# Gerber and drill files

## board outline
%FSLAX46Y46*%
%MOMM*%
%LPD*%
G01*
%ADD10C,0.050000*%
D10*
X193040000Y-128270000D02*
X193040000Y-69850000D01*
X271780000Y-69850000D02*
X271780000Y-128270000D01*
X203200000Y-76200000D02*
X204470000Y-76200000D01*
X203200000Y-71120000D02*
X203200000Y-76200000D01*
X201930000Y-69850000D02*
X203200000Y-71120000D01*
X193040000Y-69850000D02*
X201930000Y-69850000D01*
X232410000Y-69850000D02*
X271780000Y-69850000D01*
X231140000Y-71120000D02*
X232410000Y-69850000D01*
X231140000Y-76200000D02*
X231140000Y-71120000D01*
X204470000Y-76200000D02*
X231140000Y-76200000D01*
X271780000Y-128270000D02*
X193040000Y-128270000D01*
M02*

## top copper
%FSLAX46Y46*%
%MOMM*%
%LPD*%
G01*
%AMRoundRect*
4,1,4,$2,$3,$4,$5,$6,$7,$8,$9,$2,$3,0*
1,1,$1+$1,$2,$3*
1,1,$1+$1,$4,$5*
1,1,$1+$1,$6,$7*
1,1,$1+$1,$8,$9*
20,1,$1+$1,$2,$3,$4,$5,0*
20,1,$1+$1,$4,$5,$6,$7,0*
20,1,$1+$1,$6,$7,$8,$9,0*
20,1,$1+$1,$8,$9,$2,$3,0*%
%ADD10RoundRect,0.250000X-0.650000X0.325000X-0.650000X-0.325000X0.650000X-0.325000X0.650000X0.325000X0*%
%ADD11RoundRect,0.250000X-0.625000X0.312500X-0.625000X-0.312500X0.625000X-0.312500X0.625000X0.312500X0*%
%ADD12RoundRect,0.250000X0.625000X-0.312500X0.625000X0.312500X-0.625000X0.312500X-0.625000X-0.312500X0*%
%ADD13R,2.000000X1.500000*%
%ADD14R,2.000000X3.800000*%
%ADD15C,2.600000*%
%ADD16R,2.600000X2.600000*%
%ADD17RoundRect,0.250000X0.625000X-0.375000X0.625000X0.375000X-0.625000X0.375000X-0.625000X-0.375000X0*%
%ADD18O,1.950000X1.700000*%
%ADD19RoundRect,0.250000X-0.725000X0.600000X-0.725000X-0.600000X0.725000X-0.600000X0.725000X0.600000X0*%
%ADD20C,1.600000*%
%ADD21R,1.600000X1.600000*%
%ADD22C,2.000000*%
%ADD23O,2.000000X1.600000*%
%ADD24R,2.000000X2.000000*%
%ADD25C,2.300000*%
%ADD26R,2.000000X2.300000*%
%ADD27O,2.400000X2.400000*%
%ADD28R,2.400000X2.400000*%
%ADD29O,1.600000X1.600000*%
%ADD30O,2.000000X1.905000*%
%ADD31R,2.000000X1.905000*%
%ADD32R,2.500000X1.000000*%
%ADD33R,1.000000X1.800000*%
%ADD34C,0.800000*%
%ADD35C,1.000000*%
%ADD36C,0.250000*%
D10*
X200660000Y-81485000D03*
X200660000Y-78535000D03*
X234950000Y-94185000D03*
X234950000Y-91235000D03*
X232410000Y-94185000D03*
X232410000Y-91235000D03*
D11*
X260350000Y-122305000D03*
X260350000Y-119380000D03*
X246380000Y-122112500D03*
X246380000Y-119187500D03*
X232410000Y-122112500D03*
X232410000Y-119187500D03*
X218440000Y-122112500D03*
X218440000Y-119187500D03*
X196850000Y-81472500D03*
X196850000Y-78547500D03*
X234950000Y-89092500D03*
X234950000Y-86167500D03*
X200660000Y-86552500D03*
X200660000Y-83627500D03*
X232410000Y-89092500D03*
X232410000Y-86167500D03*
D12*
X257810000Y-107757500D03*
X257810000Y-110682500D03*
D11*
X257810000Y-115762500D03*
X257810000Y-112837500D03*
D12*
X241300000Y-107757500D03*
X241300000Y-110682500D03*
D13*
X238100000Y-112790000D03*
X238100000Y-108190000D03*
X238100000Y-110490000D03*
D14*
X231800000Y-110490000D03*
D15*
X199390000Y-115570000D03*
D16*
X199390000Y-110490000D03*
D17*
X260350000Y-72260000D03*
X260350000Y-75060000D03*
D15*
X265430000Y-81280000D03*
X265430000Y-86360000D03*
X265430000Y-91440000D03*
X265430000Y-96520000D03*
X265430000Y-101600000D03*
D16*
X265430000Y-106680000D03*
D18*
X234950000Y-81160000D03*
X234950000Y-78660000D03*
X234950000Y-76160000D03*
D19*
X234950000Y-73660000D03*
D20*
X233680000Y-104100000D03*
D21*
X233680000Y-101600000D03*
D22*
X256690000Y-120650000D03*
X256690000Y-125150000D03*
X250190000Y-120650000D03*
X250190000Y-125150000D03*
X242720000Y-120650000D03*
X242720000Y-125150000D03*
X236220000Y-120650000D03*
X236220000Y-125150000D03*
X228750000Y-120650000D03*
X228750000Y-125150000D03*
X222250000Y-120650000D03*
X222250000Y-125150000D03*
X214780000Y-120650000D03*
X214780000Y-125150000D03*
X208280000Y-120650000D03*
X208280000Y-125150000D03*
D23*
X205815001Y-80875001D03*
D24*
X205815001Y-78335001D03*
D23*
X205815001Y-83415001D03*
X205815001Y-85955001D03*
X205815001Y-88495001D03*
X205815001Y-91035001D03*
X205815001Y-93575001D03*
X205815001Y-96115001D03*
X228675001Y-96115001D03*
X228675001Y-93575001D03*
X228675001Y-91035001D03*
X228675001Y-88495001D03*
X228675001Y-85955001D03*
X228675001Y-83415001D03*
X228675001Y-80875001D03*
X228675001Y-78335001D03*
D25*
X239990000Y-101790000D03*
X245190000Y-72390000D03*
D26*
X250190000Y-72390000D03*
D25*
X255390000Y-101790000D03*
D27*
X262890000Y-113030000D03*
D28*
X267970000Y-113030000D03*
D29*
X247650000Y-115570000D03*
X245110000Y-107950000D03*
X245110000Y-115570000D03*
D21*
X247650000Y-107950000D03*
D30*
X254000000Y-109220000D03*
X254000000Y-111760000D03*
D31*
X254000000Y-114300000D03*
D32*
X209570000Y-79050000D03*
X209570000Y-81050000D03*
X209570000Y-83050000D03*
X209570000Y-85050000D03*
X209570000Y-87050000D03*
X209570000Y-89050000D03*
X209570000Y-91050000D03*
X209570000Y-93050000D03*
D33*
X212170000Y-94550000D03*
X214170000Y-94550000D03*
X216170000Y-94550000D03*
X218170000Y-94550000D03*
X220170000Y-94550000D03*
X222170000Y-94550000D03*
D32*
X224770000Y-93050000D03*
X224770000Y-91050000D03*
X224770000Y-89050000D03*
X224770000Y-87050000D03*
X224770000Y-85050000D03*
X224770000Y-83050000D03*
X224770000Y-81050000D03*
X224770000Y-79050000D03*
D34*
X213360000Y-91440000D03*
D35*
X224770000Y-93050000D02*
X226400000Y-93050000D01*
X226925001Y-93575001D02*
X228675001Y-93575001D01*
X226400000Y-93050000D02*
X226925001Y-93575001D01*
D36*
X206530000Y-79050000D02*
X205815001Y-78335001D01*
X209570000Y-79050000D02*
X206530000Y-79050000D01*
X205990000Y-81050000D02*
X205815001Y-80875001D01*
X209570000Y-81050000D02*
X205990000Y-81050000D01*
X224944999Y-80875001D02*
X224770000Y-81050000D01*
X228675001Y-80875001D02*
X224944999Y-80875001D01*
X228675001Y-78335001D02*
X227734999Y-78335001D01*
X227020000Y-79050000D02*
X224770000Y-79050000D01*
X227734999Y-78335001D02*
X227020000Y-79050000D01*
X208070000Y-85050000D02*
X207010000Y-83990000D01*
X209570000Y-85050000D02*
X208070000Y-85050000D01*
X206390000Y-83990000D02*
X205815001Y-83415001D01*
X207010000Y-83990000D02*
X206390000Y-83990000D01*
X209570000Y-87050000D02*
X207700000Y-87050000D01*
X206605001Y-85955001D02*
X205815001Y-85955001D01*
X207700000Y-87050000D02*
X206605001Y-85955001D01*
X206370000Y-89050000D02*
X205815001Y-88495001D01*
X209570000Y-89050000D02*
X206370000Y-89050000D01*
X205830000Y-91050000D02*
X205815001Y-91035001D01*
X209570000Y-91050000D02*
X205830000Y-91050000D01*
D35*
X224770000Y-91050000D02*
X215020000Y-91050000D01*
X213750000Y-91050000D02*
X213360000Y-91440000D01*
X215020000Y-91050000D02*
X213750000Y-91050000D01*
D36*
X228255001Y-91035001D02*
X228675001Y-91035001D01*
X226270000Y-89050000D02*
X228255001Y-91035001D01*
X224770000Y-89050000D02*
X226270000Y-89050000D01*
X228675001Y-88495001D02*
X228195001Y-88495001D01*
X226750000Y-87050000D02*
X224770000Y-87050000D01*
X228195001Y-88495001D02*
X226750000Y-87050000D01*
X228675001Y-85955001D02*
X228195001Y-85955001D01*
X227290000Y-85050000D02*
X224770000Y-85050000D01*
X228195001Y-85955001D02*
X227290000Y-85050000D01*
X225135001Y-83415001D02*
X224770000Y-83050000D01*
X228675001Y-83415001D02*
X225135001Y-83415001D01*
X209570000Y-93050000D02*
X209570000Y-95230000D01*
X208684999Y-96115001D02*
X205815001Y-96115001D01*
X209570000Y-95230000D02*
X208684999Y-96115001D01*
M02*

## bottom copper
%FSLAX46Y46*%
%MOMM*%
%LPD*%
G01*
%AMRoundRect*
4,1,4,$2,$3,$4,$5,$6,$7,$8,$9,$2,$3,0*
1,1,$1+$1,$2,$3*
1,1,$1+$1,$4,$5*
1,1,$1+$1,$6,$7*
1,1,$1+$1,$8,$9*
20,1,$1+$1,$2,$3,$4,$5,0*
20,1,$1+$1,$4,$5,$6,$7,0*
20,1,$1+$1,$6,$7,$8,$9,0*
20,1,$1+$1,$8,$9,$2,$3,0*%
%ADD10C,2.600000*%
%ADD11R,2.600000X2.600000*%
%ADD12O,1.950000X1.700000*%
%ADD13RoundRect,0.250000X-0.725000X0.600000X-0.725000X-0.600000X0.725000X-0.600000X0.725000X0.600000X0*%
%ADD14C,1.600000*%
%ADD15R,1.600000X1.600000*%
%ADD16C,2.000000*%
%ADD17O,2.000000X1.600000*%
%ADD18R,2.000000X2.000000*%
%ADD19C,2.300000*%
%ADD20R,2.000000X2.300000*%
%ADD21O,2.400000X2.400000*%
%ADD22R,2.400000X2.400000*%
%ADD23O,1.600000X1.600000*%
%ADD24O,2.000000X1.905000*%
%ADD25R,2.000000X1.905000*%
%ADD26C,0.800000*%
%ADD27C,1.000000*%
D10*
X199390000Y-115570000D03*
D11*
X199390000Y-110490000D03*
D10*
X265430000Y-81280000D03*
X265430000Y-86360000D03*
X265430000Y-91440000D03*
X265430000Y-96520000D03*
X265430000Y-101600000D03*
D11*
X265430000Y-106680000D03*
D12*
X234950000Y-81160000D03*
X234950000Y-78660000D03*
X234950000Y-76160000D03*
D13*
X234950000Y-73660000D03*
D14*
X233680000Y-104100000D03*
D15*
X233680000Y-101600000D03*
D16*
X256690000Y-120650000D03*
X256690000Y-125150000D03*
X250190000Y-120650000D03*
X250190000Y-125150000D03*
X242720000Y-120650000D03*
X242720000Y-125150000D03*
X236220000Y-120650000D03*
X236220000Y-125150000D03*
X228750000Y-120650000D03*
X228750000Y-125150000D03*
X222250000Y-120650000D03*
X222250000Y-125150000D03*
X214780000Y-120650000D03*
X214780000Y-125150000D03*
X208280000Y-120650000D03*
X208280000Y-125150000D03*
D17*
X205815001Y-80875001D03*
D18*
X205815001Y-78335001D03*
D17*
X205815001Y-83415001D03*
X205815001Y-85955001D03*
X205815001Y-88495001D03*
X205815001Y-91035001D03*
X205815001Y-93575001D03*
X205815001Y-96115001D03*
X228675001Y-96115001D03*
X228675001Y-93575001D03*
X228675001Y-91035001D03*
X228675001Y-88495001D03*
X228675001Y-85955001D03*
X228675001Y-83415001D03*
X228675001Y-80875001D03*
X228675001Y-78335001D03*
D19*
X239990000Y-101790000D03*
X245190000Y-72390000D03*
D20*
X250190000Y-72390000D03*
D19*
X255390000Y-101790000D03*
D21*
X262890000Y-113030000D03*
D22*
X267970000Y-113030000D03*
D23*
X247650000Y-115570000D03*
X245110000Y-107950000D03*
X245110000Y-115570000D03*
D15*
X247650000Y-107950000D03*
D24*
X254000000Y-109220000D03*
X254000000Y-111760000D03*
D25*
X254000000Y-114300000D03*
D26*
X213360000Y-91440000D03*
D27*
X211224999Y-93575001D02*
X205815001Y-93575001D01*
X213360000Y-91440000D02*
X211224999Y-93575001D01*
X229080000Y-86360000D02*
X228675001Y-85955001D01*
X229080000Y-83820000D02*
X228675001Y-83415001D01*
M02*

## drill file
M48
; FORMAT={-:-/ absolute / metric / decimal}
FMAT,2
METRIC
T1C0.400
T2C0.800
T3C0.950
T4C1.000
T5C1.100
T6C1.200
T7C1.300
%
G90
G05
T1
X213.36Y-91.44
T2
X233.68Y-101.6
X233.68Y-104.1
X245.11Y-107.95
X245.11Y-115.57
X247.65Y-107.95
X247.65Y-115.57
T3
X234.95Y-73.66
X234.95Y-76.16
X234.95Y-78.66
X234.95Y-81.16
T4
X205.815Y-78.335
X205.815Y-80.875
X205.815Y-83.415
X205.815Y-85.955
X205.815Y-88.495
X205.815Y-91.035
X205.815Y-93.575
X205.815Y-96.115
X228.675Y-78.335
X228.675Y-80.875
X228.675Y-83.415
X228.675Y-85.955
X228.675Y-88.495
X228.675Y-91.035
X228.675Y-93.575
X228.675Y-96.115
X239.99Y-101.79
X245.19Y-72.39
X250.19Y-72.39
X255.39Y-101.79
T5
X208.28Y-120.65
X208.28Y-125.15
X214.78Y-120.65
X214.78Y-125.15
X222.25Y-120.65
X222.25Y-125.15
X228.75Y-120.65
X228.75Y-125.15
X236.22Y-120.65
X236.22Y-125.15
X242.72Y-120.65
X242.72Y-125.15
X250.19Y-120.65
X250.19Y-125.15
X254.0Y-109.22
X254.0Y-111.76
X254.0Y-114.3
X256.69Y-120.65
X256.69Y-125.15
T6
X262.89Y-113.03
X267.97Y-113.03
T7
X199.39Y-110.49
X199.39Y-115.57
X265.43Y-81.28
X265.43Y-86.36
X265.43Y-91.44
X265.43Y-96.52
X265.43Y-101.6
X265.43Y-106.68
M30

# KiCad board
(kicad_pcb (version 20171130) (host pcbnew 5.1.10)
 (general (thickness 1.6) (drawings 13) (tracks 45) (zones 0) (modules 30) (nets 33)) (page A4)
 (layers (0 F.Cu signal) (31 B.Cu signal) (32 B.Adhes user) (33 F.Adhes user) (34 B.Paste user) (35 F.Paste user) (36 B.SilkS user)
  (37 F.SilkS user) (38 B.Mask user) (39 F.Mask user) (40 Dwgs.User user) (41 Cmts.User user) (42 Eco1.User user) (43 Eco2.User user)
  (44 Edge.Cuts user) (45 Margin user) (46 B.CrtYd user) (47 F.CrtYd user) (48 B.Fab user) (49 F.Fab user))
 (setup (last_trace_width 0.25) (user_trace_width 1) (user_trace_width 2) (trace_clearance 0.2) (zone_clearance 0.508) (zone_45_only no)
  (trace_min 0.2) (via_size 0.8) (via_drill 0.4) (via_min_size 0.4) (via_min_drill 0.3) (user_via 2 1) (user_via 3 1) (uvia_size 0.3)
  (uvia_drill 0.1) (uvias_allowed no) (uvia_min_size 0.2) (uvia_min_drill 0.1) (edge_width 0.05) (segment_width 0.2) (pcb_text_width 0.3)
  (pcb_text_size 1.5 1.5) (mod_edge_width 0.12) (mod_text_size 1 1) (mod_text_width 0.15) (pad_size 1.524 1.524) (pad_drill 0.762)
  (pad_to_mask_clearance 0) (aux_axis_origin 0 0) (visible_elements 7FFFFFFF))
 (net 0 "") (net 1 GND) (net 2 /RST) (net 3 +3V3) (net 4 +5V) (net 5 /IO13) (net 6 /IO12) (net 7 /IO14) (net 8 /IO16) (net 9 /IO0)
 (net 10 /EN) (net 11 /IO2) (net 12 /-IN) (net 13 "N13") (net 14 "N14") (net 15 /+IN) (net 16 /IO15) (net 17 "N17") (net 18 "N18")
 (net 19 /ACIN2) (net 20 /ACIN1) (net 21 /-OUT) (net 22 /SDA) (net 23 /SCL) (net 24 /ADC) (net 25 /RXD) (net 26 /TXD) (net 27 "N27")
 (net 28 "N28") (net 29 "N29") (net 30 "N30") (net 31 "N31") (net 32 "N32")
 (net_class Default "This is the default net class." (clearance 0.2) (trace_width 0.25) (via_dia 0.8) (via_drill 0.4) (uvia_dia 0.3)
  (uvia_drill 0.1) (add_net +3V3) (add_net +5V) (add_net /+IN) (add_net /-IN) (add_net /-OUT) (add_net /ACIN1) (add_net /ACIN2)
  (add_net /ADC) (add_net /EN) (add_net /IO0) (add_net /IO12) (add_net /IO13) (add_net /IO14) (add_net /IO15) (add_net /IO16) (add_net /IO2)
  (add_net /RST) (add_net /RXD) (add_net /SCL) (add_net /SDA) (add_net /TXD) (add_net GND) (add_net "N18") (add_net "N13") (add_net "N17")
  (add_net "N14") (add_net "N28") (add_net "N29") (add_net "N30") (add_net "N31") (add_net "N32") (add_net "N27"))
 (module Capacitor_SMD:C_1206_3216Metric (layer F.Cu) (at 200.66 80.01 270)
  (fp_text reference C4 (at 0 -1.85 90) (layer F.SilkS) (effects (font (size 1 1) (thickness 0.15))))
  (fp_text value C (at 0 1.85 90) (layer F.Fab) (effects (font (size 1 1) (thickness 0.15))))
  (pad 2 smd roundrect (at 1.475 0 270) (size 1.15 1.8) (layers F.Cu F.Paste F.Mask) (roundrect_rratio 0.217391) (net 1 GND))
  (pad 1 smd roundrect (at -1.475 0 270) (size 1.15 1.8) (layers F.Cu F.Paste F.Mask) (roundrect_rratio 0.217391) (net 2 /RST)))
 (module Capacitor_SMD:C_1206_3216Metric (layer F.Cu) (at 234.95 92.71 270)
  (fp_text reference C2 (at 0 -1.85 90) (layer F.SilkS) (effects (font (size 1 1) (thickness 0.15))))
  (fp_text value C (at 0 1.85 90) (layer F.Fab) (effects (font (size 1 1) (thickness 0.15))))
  (pad 2 smd roundrect (at 1.475 0 270) (size 1.15 1.8) (layers F.Cu F.Paste F.Mask) (roundrect_rratio 0.217391) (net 1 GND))
  (pad 1 smd roundrect (at -1.475 0 270) (size 1.15 1.8) (layers F.Cu F.Paste F.Mask) (roundrect_rratio 0.217391) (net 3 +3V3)))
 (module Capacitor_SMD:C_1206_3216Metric (layer F.Cu) (at 232.41 92.71 270)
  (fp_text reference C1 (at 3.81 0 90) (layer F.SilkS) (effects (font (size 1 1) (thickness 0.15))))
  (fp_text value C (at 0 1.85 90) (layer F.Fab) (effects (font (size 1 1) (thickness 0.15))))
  (pad 2 smd roundrect (at 1.475 0 270) (size 1.15 1.8) (layers F.Cu F.Paste F.Mask) (roundrect_rratio 0.217391) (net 1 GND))
  (pad 1 smd roundrect (at -1.475 0 270) (size 1.15 1.8) (layers F.Cu F.Paste F.Mask) (roundrect_rratio 0.217391) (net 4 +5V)))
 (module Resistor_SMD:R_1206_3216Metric (layer F.Cu) (at 260.35 120.8425 270)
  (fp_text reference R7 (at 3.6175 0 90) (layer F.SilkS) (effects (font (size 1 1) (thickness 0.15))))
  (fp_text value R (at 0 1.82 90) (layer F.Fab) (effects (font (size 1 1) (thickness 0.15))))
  (pad 2 smd roundrect (at 1.4625 0 270) (size 1.125 1.75) (layers F.Cu F.Paste F.Mask) (roundrect_rratio 0.222222) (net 1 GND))
  (pad 1 smd roundrect (at -1.4625 0 270) (size 1.125 1.75) (layers F.Cu F.Paste F.Mask) (roundrect_rratio 0.222222) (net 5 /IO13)))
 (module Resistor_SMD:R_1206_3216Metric (layer F.Cu) (at 246.38 120.65 270)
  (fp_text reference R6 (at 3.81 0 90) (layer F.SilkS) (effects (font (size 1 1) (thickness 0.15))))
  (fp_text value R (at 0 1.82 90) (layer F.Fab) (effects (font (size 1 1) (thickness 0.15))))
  (pad 2 smd roundrect (at 1.4625 0 270) (size 1.125 1.75) (layers F.Cu F.Paste F.Mask) (roundrect_rratio 0.222222) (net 1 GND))
  (pad 1 smd roundrect (at -1.4625 0 270) (size 1.125 1.75) (layers F.Cu F.Paste F.Mask) (roundrect_rratio 0.222222) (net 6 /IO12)))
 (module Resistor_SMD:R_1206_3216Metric (layer F.Cu) (at 232.41 120.65 270)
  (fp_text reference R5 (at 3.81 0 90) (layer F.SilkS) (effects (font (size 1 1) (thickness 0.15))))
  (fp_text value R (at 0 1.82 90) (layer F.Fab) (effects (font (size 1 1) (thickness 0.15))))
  (pad 2 smd roundrect (at 1.4625 0 270) (size 1.125 1.75) (layers F.Cu F.Paste F.Mask) (roundrect_rratio 0.222222) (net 1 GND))
  (pad 1 smd roundrect (at -1.4625 0 270) (size 1.125 1.75) (layers F.Cu F.Paste F.Mask) (roundrect_rratio 0.222222) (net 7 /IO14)))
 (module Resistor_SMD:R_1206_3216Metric (layer F.Cu) (at 218.44 120.65 270)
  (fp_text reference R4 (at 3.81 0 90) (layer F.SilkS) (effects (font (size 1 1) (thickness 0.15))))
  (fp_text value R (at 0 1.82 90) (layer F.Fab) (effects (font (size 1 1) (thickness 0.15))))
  (pad 2 smd roundrect (at 1.4625 0 270) (size 1.125 1.75) (layers F.Cu F.Paste F.Mask) (roundrect_rratio 0.222222) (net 1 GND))
  (pad 1 smd roundrect (at -1.4625 0 270) (size 1.125 1.75) (layers F.Cu F.Paste F.Mask) (roundrect_rratio 0.222222) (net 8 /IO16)))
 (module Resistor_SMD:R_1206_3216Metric (layer F.Cu) (at 196.85 80.01 270)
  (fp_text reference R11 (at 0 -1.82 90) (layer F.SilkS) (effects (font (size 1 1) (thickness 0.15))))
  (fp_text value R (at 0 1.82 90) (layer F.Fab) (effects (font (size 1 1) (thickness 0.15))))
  (pad 2 smd roundrect (at 1.4625 0 270) (size 1.125 1.75) (layers F.Cu F.Paste F.Mask) (roundrect_rratio 0.222222) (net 3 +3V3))
  (pad 1 smd roundrect (at -1.4625 0 270) (size 1.125 1.75) (layers F.Cu F.Paste F.Mask) (roundrect_rratio 0.222222) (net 2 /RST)))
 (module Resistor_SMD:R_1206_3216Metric (layer F.Cu) (at 234.95 87.63 270)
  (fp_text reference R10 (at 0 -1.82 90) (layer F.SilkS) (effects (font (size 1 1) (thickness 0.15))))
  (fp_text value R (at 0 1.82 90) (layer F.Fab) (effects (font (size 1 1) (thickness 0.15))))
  (pad 2 smd roundrect (at 1.4625 0 270) (size 1.125 1.75) (layers F.Cu F.Paste F.Mask) (roundrect_rratio 0.222222) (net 3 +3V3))
  (pad 1 smd roundrect (at -1.4625 0 270) (size 1.125 1.75) (layers F.Cu F.Paste F.Mask) (roundrect_rratio 0.222222) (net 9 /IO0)))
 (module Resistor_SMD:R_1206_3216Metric (layer F.Cu) (at 200.66 85.09 270)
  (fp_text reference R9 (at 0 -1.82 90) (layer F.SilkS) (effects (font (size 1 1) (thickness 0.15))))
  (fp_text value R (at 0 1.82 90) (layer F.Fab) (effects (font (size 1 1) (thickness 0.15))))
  (pad 2 smd roundrect (at 1.4625 0 270) (size 1.125 1.75) (layers F.Cu F.Paste F.Mask) (roundrect_rratio 0.222222) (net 3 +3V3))
  (pad 1 smd roundrect (at -1.4625 0 270) (size 1.125 1.75) (layers F.Cu F.Paste F.Mask) (roundrect_rratio 0.222222) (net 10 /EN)))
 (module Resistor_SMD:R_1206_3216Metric (layer F.Cu) (at 232.41 87.63 270)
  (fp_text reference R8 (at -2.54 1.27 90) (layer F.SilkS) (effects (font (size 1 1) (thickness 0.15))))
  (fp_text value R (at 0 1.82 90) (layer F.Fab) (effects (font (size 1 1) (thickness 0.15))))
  (pad 2 smd roundrect (at 1.4625 0 270) (size 1.125 1.75) (layers F.Cu F.Paste F.Mask) (roundrect_rratio 0.222222) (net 3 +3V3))
  (pad 1 smd roundrect (at -1.4625 0 270) (size 1.125 1.75) (layers F.Cu F.Paste F.Mask) (roundrect_rratio 0.222222) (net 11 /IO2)))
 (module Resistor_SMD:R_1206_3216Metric (layer F.Cu) (at 257.81 109.22 90)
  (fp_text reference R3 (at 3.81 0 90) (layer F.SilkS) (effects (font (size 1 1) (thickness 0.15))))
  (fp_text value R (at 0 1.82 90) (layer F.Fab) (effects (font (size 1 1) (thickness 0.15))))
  (pad 2 smd roundrect (at 1.4625 0 90) (size 1.125 1.75) (layers F.Cu F.Paste F.Mask) (roundrect_rratio 0.222222) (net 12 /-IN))
  (pad 1 smd roundrect (at -1.4625 0 90) (size 1.125 1.75) (layers F.Cu F.Paste F.Mask) (roundrect_rratio 0.222222) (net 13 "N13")))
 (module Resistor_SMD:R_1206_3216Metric (layer F.Cu) (at 257.81 114.3 270)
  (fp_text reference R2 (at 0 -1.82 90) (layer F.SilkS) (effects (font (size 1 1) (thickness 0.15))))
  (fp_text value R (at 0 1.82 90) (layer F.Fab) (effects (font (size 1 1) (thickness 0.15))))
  (pad 2 smd roundrect (at 1.4625 0 270) (size 1.125 1.75) (layers F.Cu F.Paste F.Mask) (roundrect_rratio 0.222222) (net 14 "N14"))
  (pad 1 smd roundrect (at -1.4625 0 270) (size 1.125 1.75) (layers F.Cu F.Paste F.Mask) (roundrect_rratio 0.222222) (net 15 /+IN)))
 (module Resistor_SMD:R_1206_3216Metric (layer F.Cu) (at 241.3 109.22 90)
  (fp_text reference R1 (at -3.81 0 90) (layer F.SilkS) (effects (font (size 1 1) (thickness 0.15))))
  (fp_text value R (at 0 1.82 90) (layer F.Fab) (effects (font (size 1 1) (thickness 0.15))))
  (pad 2 smd roundrect (at 1.4625 0 90) (size 1.125 1.75) (layers F.Cu F.Paste F.Mask) (roundrect_rratio 0.222222) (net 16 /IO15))
  (pad 1 smd roundrect (at -1.4625 0 90) (size 1.125 1.75) (layers F.Cu F.Paste F.Mask) (roundrect_rratio 0.222222) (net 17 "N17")))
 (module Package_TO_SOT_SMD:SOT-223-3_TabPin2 (layer F.Cu) (at 234.95 110.49 180)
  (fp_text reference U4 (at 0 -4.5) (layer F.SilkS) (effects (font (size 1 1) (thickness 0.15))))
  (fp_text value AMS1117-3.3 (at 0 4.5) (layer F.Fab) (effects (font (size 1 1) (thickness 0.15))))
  (pad 1 smd rect (at -3.15 -2.3 180) (size 2 1.5) (layers F.Cu F.Paste F.Mask) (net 1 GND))
  (pad 3 smd rect (at -3.15 2.3 180) (size 2 1.5) (layers F.Cu F.Paste F.Mask) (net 4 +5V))
  (pad 2 smd rect (at -3.15 0 180) (size 2 1.5) (layers F.Cu F.Paste F.Mask) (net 3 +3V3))
  (pad 2 smd rect (at 3.15 0 180) (size 2 3.8) (layers F.Cu F.Paste F.Mask) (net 3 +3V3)))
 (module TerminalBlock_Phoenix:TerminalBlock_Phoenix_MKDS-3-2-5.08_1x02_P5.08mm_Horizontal (layer F.Cu) (at 199.39 110.49 270)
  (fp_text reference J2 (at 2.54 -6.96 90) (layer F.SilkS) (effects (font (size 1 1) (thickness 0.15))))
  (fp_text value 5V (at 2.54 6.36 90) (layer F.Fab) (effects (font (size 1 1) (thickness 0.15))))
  (pad 2 thru_hole circle (at 5.08 0 270) (size 2.6 2.6) (drill 1.3) (layers *.Cu *.Mask) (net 1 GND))
  (pad 1 thru_hole rect (at 0 0 270) (size 2.6 2.6) (drill 1.3) (layers *.Cu *.Mask) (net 4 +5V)))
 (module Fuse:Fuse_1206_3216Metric (layer F.Cu) (at 260.35 73.66 90)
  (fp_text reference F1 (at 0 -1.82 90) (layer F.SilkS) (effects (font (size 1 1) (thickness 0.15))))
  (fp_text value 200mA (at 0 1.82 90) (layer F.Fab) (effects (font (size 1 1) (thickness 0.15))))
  (pad 2 smd roundrect (at 1.4 0 90) (size 1.25 1.75) (layers F.Cu F.Paste F.Mask) (roundrect_rratio 0.2) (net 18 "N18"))
  (pad 1 smd roundrect (at -1.4 0 90) (size 1.25 1.75) (layers F.Cu F.Paste F.Mask) (roundrect_rratio 0.2) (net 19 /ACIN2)))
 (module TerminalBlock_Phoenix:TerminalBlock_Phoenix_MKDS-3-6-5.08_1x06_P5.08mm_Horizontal (layer F.Cu) (at 265.43 106.68 90)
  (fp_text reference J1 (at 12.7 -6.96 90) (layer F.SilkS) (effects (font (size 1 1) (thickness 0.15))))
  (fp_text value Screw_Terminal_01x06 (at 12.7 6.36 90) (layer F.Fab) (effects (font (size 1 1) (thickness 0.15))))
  (pad 6 thru_hole circle (at 25.4 0 90) (size 2.6 2.6) (drill 1.3) (layers *.Cu *.Mask) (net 19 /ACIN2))
  (pad 5 thru_hole circle (at 20.32 0 90) (size 2.6 2.6) (drill 1.3) (layers *.Cu *.Mask) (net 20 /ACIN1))
  (pad 4 thru_hole circle (at 15.24 0 90) (size 2.6 2.6) (drill 1.3) (layers *.Cu *.Mask) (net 12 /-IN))
  (pad 3 thru_hole circle (at 10.16 0 90) (size 2.6 2.6) (drill 1.3) (layers *.Cu *.Mask) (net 15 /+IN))
  (pad 2 thru_hole circle (at 5.08 0 90) (size 2.6 2.6) (drill 1.3) (layers *.Cu *.Mask) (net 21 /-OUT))
  (pad 1 thru_hole rect (at 0 0 90) (size 2.6 2.6) (drill 1.3) (layers *.Cu *.Mask) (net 15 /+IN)))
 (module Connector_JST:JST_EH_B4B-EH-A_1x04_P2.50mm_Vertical (layer F.Cu) (at 234.95 73.66 270)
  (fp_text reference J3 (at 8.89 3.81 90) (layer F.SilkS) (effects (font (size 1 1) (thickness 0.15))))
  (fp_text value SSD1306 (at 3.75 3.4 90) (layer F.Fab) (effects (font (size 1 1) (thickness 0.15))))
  (pad 4 thru_hole oval (at 7.5 0 270) (size 1.7 1.95) (drill 0.95) (layers *.Cu *.Mask) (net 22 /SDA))
  (pad 3 thru_hole oval (at 5 0 270) (size 1.7 1.95) (drill 0.95) (layers *.Cu *.Mask) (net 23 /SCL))
  (pad 2 thru_hole oval (at 2.5 0 270) (size 1.7 1.95) (drill 0.95) (layers *.Cu *.Mask) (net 4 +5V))
  (pad 1 thru_hole roundrect (at 0 0 270) (size 1.7 1.95) (drill 0.95) (layers *.Cu *.Mask) (roundrect_rratio 0.147059) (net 1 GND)))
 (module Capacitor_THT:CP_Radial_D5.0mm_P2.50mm (layer F.Cu) (at 233.68 101.6 270)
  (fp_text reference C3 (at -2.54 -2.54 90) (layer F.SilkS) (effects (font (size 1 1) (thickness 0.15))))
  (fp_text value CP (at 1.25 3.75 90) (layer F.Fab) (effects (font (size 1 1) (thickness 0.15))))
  (pad 2 thru_hole circle (at 2.5 0 270) (size 1.6 1.6) (drill 0.8) (layers *.Cu *.Mask) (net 1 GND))
  (pad 1 thru_hole rect (at 0 0 270) (size 1.6 1.6) (drill 0.8) (layers *.Cu *.Mask) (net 3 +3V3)))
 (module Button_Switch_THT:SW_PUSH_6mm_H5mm (layer F.Cu) (at 250.19 120.65)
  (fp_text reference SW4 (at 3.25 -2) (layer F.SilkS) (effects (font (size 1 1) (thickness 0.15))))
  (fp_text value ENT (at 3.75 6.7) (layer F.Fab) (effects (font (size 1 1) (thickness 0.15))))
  (pad 1 thru_hole circle (at 6.5 0 90) (size 2 2) (drill 1.1) (layers *.Cu *.Mask) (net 5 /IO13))
  (pad 2 thru_hole circle (at 6.5 4.5 90) (size 2 2) (drill 1.1) (layers *.Cu *.Mask) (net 3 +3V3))
  (pad 1 thru_hole circle (at 0 0 90) (size 2 2) (drill 1.1) (layers *.Cu *.Mask) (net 5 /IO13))
  (pad 2 thru_hole circle (at 0 4.5 90) (size 2 2) (drill 1.1) (layers *.Cu *.Mask) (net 3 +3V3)))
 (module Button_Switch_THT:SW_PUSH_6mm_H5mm (layer F.Cu) (at 236.22 120.65)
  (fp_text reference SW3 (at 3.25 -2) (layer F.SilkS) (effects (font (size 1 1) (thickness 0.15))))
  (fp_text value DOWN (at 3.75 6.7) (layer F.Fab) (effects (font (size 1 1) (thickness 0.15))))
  (pad 1 thru_hole circle (at 6.5 0 90) (size 2 2) (drill 1.1) (layers *.Cu *.Mask) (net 6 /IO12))
  (pad 2 thru_hole circle (at 6.5 4.5 90) (size 2 2) (drill 1.1) (layers *.Cu *.Mask) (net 3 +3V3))
  (pad 1 thru_hole circle (at 0 0 90) (size 2 2) (drill 1.1) (layers *.Cu *.Mask) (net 6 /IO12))
  (pad 2 thru_hole circle (at 0 4.5 90) (size 2 2) (drill 1.1) (layers *.Cu *.Mask) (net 3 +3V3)))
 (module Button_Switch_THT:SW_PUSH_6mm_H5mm (layer F.Cu) (at 222.25 120.65)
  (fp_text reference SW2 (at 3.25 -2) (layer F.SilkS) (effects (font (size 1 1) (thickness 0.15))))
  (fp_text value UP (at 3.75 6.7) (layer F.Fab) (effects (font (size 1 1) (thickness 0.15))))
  (pad 1 thru_hole circle (at 6.5 0 90) (size 2 2) (drill 1.1) (layers *.Cu *.Mask) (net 7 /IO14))
  (pad 2 thru_hole circle (at 6.5 4.5 90) (size 2 2) (drill 1.1) (layers *.Cu *.Mask) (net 3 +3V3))
  (pad 1 thru_hole circle (at 0 0 90) (size 2 2) (drill 1.1) (layers *.Cu *.Mask) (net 7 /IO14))
  (pad 2 thru_hole circle (at 0 4.5 90) (size 2 2) (drill 1.1) (layers *.Cu *.Mask) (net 3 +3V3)))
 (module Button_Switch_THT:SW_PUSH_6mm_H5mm (layer F.Cu) (at 208.28 120.65)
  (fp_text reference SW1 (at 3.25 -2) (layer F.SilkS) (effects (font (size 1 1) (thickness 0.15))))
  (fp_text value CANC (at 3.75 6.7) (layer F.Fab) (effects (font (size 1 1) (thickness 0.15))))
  (pad 1 thru_hole circle (at 6.5 0 90) (size 2 2) (drill 1.1) (layers *.Cu *.Mask) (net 8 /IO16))
  (pad 2 thru_hole circle (at 6.5 4.5 90) (size 2 2) (drill 1.1) (layers *.Cu *.Mask) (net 3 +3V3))
  (pad 1 thru_hole circle (at 0 0 90) (size 2 2) (drill 1.1) (layers *.Cu *.Mask) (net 8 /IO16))
  (pad 2 thru_hole circle (at 0 4.5 90) (size 2 2) (drill 1.1) (layers *.Cu *.Mask) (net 3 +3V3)))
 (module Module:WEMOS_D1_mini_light (layer F.Cu) (at 205.815001 78.335001)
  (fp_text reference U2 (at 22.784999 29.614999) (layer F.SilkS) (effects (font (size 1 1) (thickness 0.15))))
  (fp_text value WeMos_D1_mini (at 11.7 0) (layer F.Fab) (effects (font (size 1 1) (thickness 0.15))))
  (pad 2 thru_hole oval (at 0 2.54) (size 2 1.6) (drill 1) (layers *.Cu *.Mask) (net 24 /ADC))
  (pad 1 thru_hole rect (at 0 0) (size 2 2) (drill 1) (layers *.Cu *.Mask) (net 2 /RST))
  (pad 3 thru_hole oval (at 0 5.08) (size 2 1.6) (drill 1) (layers *.Cu *.Mask) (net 8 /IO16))
  (pad 4 thru_hole oval (at 0 7.62) (size 2 1.6) (drill 1) (layers *.Cu *.Mask) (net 7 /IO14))
  (pad 5 thru_hole oval (at 0 10.16) (size 2 1.6) (drill 1) (layers *.Cu *.Mask) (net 6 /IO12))
  (pad 6 thru_hole oval (at 0 12.7) (size 2 1.6) (drill 1) (layers *.Cu *.Mask) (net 5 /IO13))
  (pad 7 thru_hole oval (at 0 15.24) (size 2 1.6) (drill 1) (layers *.Cu *.Mask) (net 16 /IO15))
  (pad 8 thru_hole oval (at 0 17.78) (size 2 1.6) (drill 1) (layers *.Cu *.Mask) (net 3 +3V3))
  (pad 9 thru_hole oval (at 22.86 17.78) (size 2 1.6) (drill 1) (layers *.Cu *.Mask) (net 4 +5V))
  (pad 10 thru_hole oval (at 22.86 15.24) (size 2 1.6) (drill 1) (layers *.Cu *.Mask) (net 1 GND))
  (pad 11 thru_hole oval (at 22.86 12.7) (size 2 1.6) (drill 1) (layers *.Cu *.Mask) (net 11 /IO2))
  (pad 12 thru_hole oval (at 22.86 10.16) (size 2 1.6) (drill 1) (layers *.Cu *.Mask) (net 9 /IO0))
  (pad 13 thru_hole oval (at 22.86 7.62) (size 2 1.6) (drill 1) (layers *.Cu *.Mask) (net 22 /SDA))
  (pad 14 thru_hole oval (at 22.86 5.08) (size 2 1.6) (drill 1) (layers *.Cu *.Mask) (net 23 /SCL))
  (pad 15 thru_hole oval (at 22.86 2.54) (size 2 1.6) (drill 1) (layers *.Cu *.Mask) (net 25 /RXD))
  (pad 16 thru_hole oval (at 22.86 0) (size 2 1.6) (drill 1) (layers *.Cu *.Mask) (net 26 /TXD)))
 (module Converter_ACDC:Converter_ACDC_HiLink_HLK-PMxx (layer F.Cu) (at 250.19 72.39 270)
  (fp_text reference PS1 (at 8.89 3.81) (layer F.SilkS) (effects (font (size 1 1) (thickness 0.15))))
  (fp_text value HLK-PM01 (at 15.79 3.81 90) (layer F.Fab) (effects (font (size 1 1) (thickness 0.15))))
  (pad 4 thru_hole circle (at 29.4 10.2 270) (size 2.3 2.3) (drill 1) (layers *.Cu *.Mask) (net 4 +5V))
  (pad 2 thru_hole circle (at 0 5 270) (size 2.3 2.3) (drill 1) (layers *.Cu *.Mask) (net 20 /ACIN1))
  (pad 1 thru_hole rect (at 0 0 270) (size 2.3 2) (drill 1) (layers *.Cu *.Mask) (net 18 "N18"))
  (pad 3 thru_hole circle (at 29.4 -5.2 270) (size 2.3 2.3) (drill 1) (layers *.Cu *.Mask) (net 1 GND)))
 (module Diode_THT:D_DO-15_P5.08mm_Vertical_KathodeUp (layer F.Cu) (at 267.97 113.03 180)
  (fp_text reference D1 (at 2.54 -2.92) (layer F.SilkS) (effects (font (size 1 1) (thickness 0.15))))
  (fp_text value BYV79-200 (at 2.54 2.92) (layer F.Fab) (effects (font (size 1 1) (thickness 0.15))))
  (pad 2 thru_hole oval (at 5.08 0 180) (size 2.4 2.4) (drill 1.2) (layers *.Cu *.Mask) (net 21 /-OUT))
  (pad 1 thru_hole rect (at 0 0 180) (size 2.4 2.4) (drill 1.2) (layers *.Cu *.Mask) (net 15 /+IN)))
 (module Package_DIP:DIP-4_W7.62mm (layer F.Cu) (at 247.65 107.95 270)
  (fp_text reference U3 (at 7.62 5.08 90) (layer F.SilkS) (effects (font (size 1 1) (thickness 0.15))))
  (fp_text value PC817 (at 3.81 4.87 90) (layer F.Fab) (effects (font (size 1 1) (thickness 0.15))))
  (pad 4 thru_hole oval (at 7.62 0 270) (size 1.6 1.6) (drill 0.8) (layers *.Cu *.Mask) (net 14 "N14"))
  (pad 2 thru_hole oval (at 0 2.54 270) (size 1.6 1.6) (drill 0.8) (layers *.Cu *.Mask) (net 1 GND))
  (pad 3 thru_hole oval (at 7.62 2.54 270) (size 1.6 1.6) (drill 0.8) (layers *.Cu *.Mask) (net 13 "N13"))
  (pad 1 thru_hole rect (at 0 0 270) (size 1.6 1.6) (drill 0.8) (layers *.Cu *.Mask) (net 17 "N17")))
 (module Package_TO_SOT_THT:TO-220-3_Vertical (layer F.Cu) (at 254 114.3 90)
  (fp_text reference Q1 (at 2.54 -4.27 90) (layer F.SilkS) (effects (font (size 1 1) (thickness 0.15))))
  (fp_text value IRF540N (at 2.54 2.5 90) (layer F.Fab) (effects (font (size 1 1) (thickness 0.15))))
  (pad 3 thru_hole oval (at 5.08 0 90) (size 1.905 2) (drill 1.1) (layers *.Cu *.Mask) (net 12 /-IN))
  (pad 2 thru_hole oval (at 2.54 0 90) (size 1.905 2) (drill 1.1) (layers *.Cu *.Mask) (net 21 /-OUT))
  (pad 1 thru_hole rect (at 0 0 90) (size 1.905 2) (drill 1.1) (layers *.Cu *.Mask) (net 13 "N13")))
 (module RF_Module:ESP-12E (layer F.Cu) (at 217.17 82.55)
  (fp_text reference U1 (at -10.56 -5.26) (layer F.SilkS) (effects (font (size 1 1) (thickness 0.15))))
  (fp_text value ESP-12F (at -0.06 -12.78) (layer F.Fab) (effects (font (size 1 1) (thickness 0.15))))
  (pad 1 smd rect (at -7.6 -3.5) (size 2.5 1) (layers F.Cu F.Paste F.Mask) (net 2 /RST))
  (pad 2 smd rect (at -7.6 -1.5) (size 2.5 1) (layers F.Cu F.Paste F.Mask) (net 24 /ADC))
  (pad 3 smd rect (at -7.6 0.5) (size 2.5 1) (layers F.Cu F.Paste F.Mask) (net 10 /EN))
  (pad 4 smd rect (at -7.6 2.5) (size 2.5 1) (layers F.Cu F.Paste F.Mask) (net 8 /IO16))
  (pad 5 smd rect (at -7.6 4.5) (size 2.5 1) (layers F.Cu F.Paste F.Mask) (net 7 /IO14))
  (pad 6 smd rect (at -7.6 6.5) (size 2.5 1) (layers F.Cu F.Paste F.Mask) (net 6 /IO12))
  (pad 7 smd rect (at -7.6 8.5) (size 2.5 1) (layers F.Cu F.Paste F.Mask) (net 5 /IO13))
  (pad 8 smd rect (at -7.6 10.5) (size 2.5 1) (layers F.Cu F.Paste F.Mask) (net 3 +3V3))
  (pad 9 smd rect (at -5 12) (size 1 1.8) (layers F.Cu F.Paste F.Mask) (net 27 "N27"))
  (pad 10 smd rect (at -3 12) (size 1 1.8) (layers F.Cu F.Paste F.Mask) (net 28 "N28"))
  (pad 11 smd rect (at -1 12) (size 1 1.8) (layers F.Cu F.Paste F.Mask) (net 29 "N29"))
  (pad 12 smd rect (at 1 12) (size 1 1.8) (layers F.Cu F.Paste F.Mask) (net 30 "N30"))
  (pad 13 smd rect (at 3 12) (size 1 1.8) (layers F.Cu F.Paste F.Mask) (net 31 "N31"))
  (pad 14 smd rect (at 5 12) (size 1 1.8) (layers F.Cu F.Paste F.Mask) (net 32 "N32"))
  (pad 15 smd rect (at 7.6 10.5) (size 2.5 1) (layers F.Cu F.Paste F.Mask) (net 1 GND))
  (pad 16 smd rect (at 7.6 8.5) (size 2.5 1) (layers F.Cu F.Paste F.Mask) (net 16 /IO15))
  (pad 17 smd rect (at 7.6 6.5) (size 2.5 1) (layers F.Cu F.Paste F.Mask) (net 11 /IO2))
  (pad 18 smd rect (at 7.6 4.5) (size 2.5 1) (layers F.Cu F.Paste F.Mask) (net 9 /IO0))
  (pad 19 smd rect (at 7.6 2.5) (size 2.5 1) (layers F.Cu F.Paste F.Mask) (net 22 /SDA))
  (pad 20 smd rect (at 7.6 0.5) (size 2.5 1) (layers F.Cu F.Paste F.Mask) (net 23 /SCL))
  (pad 21 smd rect (at 7.6 -1.5) (size 2.5 1) (layers F.Cu F.Paste F.Mask) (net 25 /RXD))
  (pad 22 smd rect (at 7.6 -3.5) (size 2.5 1) (layers F.Cu F.Paste F.Mask) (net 26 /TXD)))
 (gr_line (start 193.04 128.27) (end 193.04 69.85) (layer Edge.Cuts) (width 0.05))
 (gr_line (start 271.78 69.85) (end 271.78 128.27) (layer Edge.Cuts) (width 0.05))
 (gr_line (start 203.2 76.2) (end 204.47 76.2) (layer Edge.Cuts) (width 0.05))
 (gr_line (start 203.2 71.12) (end 203.2 76.2) (layer Edge.Cuts) (width 0.05))
 (gr_line (start 201.93 69.85) (end 203.2 71.12) (layer Edge.Cuts) (width 0.05))
 (gr_line (start 193.04 69.85) (end 201.93 69.85) (layer Edge.Cuts) (width 0.05))
 (gr_line (start 232.41 69.85) (end 271.78 69.85) (layer Edge.Cuts) (width 0.05))
 (gr_line (start 231.14 71.12) (end 232.41 69.85) (layer Edge.Cuts) (width 0.05))
 (gr_line (start 231.14 76.2) (end 231.14 71.12) (layer Edge.Cuts) (width 0.05))
 (gr_line (start 204.47 76.2) (end 231.14 76.2) (layer Edge.Cuts) (width 0.05))
 (gr_line (start 271.78 128.27) (end 193.04 128.27) (layer Edge.Cuts) (width 0.05))
 (segment (start 224.77 93.05) (end 226.4 93.05) (width 1) (layer F.Cu) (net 1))
 (segment (start 226.925001 93.575001) (end 228.675001 93.575001) (width 1) (layer F.Cu) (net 1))
 (segment (start 226.4 93.05) (end 226.925001 93.575001) (width 1) (layer F.Cu) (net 1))
 (segment (start 206.53 79.05) (end 205.815001 78.335001) (width 0.25) (layer F.Cu) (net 2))
 (segment (start 209.57 79.05) (end 206.53 79.05) (width 0.25) (layer F.Cu) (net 2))
 (segment (start 205.99 81.05) (end 205.815001 80.875001) (width 0.25) (layer F.Cu) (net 24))
 (segment (start 209.57 81.05) (end 205.99 81.05) (width 0.25) (layer F.Cu) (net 24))
 (segment (start 224.944999 80.875001) (end 224.77 81.05) (width 0.25) (layer F.Cu) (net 25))
 (segment (start 228.675001 80.875001) (end 224.944999 80.875001) (width 0.25) (layer F.Cu) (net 25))
 (segment (start 228.675001 78.335001) (end 227.734999 78.335001) (width 0.25) (layer F.Cu) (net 26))
 (segment (start 227.02 79.05) (end 224.77 79.05) (width 0.25) (layer F.Cu) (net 26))
 (segment (start 227.734999 78.335001) (end 227.02 79.05) (width 0.25) (layer F.Cu) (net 26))
 (segment (start 208.07 85.05) (end 207.01 83.99) (width 0.25) (layer F.Cu) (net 8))
 (segment (start 209.57 85.05) (end 208.07 85.05) (width 0.25) (layer F.Cu) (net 8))
 (segment (start 206.39 83.99) (end 205.815001 83.415001) (width 0.25) (layer F.Cu) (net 8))
 (segment (start 207.01 83.99) (end 206.39 83.99) (width 0.25) (layer F.Cu) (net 8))
 (segment (start 209.57 87.05) (end 207.7 87.05) (width 0.25) (layer F.Cu) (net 7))
 (segment (start 206.605001 85.955001) (end 205.815001 85.955001) (width 0.25) (layer F.Cu) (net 7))
 (segment (start 207.7 87.05) (end 206.605001 85.955001) (width 0.25) (layer F.Cu) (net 7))
 (segment (start 206.37 89.05) (end 205.815001 88.495001) (width 0.25) (layer F.Cu) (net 6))
 (segment (start 209.57 89.05) (end 206.37 89.05) (width 0.25) (layer F.Cu) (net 6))
 (segment (start 205.83 91.05) (end 205.815001 91.035001) (width 0.25) (layer F.Cu) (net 5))
 (segment (start 209.57 91.05) (end 205.83 91.05) (width 0.25) (layer F.Cu) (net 5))
 (segment (start 224.77 91.05) (end 215.02 91.05) (width 1) (layer F.Cu) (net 16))
 (via (at 213.36 91.44) (size 0.8) (drill 0.4) (layers F.Cu B.Cu) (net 16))
 (segment (start 213.75 91.05) (end 213.36 91.44) (width 1) (layer F.Cu) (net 16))
 (segment (start 215.02 91.05) (end 213.75 91.05) (width 1) (layer F.Cu) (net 16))
 (segment (start 211.224999 93.575001) (end 205.815001 93.575001) (width 1) (layer B.Cu) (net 16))
 (segment (start 213.36 91.44) (end 211.224999 93.575001) (width 1) (layer B.Cu) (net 16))
 (segment (start 228.255001 91.035001) (end 228.675001 91.035001) (width 0.25) (layer F.Cu) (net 11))
 (segment (start 226.27 89.05) (end 228.255001 91.035001) (width 0.25) (layer F.Cu) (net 11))
 (segment (start 224.77 89.05) (end 226.27 89.05) (width 0.25) (layer F.Cu) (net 11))
 (segment (start 228.675001 88.495001) (end 228.195001 88.495001) (width 0.25) (layer F.Cu) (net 9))
 (segment (start 226.75 87.05) (end 224.77 87.05) (width 0.25) (layer F.Cu) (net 9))
 (segment (start 228.195001 88.495001) (end 226.75 87.05) (width 0.25) (layer F.Cu) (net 9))
 (segment (start 228.675001 85.955001) (end 228.195001 85.955001) (width 0.25) (layer F.Cu) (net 22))
 (segment (start 227.29 85.05) (end 224.77 85.05) (width 0.25) (layer F.Cu) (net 22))
 (segment (start 228.195001 85.955001) (end 227.29 85.05) (width 0.25) (layer F.Cu) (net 22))
 (segment (start 229.08 86.36) (end 228.675001 85.955001) (width 1) (layer B.Cu) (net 22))
 (segment (start 225.135001 83.415001) (end 224.77 83.05) (width 0.25) (layer F.Cu) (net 23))
 (segment (start 228.675001 83.415001) (end 225.135001 83.415001) (width 0.25) (layer F.Cu) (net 23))
 (segment (start 229.08 83.82) (end 228.675001 83.415001) (width 1) (layer B.Cu) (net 23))
 (segment (start 209.57 93.05) (end 209.57 95.23) (width 0.25) (layer F.Cu) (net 3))
 (segment (start 208.684999 96.115001) (end 205.815001 96.115001) (width 0.25) (layer F.Cu) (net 3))
 (segment (start 209.57 95.23) (end 208.684999 96.115001) (width 0.25) (layer F.Cu) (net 3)))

